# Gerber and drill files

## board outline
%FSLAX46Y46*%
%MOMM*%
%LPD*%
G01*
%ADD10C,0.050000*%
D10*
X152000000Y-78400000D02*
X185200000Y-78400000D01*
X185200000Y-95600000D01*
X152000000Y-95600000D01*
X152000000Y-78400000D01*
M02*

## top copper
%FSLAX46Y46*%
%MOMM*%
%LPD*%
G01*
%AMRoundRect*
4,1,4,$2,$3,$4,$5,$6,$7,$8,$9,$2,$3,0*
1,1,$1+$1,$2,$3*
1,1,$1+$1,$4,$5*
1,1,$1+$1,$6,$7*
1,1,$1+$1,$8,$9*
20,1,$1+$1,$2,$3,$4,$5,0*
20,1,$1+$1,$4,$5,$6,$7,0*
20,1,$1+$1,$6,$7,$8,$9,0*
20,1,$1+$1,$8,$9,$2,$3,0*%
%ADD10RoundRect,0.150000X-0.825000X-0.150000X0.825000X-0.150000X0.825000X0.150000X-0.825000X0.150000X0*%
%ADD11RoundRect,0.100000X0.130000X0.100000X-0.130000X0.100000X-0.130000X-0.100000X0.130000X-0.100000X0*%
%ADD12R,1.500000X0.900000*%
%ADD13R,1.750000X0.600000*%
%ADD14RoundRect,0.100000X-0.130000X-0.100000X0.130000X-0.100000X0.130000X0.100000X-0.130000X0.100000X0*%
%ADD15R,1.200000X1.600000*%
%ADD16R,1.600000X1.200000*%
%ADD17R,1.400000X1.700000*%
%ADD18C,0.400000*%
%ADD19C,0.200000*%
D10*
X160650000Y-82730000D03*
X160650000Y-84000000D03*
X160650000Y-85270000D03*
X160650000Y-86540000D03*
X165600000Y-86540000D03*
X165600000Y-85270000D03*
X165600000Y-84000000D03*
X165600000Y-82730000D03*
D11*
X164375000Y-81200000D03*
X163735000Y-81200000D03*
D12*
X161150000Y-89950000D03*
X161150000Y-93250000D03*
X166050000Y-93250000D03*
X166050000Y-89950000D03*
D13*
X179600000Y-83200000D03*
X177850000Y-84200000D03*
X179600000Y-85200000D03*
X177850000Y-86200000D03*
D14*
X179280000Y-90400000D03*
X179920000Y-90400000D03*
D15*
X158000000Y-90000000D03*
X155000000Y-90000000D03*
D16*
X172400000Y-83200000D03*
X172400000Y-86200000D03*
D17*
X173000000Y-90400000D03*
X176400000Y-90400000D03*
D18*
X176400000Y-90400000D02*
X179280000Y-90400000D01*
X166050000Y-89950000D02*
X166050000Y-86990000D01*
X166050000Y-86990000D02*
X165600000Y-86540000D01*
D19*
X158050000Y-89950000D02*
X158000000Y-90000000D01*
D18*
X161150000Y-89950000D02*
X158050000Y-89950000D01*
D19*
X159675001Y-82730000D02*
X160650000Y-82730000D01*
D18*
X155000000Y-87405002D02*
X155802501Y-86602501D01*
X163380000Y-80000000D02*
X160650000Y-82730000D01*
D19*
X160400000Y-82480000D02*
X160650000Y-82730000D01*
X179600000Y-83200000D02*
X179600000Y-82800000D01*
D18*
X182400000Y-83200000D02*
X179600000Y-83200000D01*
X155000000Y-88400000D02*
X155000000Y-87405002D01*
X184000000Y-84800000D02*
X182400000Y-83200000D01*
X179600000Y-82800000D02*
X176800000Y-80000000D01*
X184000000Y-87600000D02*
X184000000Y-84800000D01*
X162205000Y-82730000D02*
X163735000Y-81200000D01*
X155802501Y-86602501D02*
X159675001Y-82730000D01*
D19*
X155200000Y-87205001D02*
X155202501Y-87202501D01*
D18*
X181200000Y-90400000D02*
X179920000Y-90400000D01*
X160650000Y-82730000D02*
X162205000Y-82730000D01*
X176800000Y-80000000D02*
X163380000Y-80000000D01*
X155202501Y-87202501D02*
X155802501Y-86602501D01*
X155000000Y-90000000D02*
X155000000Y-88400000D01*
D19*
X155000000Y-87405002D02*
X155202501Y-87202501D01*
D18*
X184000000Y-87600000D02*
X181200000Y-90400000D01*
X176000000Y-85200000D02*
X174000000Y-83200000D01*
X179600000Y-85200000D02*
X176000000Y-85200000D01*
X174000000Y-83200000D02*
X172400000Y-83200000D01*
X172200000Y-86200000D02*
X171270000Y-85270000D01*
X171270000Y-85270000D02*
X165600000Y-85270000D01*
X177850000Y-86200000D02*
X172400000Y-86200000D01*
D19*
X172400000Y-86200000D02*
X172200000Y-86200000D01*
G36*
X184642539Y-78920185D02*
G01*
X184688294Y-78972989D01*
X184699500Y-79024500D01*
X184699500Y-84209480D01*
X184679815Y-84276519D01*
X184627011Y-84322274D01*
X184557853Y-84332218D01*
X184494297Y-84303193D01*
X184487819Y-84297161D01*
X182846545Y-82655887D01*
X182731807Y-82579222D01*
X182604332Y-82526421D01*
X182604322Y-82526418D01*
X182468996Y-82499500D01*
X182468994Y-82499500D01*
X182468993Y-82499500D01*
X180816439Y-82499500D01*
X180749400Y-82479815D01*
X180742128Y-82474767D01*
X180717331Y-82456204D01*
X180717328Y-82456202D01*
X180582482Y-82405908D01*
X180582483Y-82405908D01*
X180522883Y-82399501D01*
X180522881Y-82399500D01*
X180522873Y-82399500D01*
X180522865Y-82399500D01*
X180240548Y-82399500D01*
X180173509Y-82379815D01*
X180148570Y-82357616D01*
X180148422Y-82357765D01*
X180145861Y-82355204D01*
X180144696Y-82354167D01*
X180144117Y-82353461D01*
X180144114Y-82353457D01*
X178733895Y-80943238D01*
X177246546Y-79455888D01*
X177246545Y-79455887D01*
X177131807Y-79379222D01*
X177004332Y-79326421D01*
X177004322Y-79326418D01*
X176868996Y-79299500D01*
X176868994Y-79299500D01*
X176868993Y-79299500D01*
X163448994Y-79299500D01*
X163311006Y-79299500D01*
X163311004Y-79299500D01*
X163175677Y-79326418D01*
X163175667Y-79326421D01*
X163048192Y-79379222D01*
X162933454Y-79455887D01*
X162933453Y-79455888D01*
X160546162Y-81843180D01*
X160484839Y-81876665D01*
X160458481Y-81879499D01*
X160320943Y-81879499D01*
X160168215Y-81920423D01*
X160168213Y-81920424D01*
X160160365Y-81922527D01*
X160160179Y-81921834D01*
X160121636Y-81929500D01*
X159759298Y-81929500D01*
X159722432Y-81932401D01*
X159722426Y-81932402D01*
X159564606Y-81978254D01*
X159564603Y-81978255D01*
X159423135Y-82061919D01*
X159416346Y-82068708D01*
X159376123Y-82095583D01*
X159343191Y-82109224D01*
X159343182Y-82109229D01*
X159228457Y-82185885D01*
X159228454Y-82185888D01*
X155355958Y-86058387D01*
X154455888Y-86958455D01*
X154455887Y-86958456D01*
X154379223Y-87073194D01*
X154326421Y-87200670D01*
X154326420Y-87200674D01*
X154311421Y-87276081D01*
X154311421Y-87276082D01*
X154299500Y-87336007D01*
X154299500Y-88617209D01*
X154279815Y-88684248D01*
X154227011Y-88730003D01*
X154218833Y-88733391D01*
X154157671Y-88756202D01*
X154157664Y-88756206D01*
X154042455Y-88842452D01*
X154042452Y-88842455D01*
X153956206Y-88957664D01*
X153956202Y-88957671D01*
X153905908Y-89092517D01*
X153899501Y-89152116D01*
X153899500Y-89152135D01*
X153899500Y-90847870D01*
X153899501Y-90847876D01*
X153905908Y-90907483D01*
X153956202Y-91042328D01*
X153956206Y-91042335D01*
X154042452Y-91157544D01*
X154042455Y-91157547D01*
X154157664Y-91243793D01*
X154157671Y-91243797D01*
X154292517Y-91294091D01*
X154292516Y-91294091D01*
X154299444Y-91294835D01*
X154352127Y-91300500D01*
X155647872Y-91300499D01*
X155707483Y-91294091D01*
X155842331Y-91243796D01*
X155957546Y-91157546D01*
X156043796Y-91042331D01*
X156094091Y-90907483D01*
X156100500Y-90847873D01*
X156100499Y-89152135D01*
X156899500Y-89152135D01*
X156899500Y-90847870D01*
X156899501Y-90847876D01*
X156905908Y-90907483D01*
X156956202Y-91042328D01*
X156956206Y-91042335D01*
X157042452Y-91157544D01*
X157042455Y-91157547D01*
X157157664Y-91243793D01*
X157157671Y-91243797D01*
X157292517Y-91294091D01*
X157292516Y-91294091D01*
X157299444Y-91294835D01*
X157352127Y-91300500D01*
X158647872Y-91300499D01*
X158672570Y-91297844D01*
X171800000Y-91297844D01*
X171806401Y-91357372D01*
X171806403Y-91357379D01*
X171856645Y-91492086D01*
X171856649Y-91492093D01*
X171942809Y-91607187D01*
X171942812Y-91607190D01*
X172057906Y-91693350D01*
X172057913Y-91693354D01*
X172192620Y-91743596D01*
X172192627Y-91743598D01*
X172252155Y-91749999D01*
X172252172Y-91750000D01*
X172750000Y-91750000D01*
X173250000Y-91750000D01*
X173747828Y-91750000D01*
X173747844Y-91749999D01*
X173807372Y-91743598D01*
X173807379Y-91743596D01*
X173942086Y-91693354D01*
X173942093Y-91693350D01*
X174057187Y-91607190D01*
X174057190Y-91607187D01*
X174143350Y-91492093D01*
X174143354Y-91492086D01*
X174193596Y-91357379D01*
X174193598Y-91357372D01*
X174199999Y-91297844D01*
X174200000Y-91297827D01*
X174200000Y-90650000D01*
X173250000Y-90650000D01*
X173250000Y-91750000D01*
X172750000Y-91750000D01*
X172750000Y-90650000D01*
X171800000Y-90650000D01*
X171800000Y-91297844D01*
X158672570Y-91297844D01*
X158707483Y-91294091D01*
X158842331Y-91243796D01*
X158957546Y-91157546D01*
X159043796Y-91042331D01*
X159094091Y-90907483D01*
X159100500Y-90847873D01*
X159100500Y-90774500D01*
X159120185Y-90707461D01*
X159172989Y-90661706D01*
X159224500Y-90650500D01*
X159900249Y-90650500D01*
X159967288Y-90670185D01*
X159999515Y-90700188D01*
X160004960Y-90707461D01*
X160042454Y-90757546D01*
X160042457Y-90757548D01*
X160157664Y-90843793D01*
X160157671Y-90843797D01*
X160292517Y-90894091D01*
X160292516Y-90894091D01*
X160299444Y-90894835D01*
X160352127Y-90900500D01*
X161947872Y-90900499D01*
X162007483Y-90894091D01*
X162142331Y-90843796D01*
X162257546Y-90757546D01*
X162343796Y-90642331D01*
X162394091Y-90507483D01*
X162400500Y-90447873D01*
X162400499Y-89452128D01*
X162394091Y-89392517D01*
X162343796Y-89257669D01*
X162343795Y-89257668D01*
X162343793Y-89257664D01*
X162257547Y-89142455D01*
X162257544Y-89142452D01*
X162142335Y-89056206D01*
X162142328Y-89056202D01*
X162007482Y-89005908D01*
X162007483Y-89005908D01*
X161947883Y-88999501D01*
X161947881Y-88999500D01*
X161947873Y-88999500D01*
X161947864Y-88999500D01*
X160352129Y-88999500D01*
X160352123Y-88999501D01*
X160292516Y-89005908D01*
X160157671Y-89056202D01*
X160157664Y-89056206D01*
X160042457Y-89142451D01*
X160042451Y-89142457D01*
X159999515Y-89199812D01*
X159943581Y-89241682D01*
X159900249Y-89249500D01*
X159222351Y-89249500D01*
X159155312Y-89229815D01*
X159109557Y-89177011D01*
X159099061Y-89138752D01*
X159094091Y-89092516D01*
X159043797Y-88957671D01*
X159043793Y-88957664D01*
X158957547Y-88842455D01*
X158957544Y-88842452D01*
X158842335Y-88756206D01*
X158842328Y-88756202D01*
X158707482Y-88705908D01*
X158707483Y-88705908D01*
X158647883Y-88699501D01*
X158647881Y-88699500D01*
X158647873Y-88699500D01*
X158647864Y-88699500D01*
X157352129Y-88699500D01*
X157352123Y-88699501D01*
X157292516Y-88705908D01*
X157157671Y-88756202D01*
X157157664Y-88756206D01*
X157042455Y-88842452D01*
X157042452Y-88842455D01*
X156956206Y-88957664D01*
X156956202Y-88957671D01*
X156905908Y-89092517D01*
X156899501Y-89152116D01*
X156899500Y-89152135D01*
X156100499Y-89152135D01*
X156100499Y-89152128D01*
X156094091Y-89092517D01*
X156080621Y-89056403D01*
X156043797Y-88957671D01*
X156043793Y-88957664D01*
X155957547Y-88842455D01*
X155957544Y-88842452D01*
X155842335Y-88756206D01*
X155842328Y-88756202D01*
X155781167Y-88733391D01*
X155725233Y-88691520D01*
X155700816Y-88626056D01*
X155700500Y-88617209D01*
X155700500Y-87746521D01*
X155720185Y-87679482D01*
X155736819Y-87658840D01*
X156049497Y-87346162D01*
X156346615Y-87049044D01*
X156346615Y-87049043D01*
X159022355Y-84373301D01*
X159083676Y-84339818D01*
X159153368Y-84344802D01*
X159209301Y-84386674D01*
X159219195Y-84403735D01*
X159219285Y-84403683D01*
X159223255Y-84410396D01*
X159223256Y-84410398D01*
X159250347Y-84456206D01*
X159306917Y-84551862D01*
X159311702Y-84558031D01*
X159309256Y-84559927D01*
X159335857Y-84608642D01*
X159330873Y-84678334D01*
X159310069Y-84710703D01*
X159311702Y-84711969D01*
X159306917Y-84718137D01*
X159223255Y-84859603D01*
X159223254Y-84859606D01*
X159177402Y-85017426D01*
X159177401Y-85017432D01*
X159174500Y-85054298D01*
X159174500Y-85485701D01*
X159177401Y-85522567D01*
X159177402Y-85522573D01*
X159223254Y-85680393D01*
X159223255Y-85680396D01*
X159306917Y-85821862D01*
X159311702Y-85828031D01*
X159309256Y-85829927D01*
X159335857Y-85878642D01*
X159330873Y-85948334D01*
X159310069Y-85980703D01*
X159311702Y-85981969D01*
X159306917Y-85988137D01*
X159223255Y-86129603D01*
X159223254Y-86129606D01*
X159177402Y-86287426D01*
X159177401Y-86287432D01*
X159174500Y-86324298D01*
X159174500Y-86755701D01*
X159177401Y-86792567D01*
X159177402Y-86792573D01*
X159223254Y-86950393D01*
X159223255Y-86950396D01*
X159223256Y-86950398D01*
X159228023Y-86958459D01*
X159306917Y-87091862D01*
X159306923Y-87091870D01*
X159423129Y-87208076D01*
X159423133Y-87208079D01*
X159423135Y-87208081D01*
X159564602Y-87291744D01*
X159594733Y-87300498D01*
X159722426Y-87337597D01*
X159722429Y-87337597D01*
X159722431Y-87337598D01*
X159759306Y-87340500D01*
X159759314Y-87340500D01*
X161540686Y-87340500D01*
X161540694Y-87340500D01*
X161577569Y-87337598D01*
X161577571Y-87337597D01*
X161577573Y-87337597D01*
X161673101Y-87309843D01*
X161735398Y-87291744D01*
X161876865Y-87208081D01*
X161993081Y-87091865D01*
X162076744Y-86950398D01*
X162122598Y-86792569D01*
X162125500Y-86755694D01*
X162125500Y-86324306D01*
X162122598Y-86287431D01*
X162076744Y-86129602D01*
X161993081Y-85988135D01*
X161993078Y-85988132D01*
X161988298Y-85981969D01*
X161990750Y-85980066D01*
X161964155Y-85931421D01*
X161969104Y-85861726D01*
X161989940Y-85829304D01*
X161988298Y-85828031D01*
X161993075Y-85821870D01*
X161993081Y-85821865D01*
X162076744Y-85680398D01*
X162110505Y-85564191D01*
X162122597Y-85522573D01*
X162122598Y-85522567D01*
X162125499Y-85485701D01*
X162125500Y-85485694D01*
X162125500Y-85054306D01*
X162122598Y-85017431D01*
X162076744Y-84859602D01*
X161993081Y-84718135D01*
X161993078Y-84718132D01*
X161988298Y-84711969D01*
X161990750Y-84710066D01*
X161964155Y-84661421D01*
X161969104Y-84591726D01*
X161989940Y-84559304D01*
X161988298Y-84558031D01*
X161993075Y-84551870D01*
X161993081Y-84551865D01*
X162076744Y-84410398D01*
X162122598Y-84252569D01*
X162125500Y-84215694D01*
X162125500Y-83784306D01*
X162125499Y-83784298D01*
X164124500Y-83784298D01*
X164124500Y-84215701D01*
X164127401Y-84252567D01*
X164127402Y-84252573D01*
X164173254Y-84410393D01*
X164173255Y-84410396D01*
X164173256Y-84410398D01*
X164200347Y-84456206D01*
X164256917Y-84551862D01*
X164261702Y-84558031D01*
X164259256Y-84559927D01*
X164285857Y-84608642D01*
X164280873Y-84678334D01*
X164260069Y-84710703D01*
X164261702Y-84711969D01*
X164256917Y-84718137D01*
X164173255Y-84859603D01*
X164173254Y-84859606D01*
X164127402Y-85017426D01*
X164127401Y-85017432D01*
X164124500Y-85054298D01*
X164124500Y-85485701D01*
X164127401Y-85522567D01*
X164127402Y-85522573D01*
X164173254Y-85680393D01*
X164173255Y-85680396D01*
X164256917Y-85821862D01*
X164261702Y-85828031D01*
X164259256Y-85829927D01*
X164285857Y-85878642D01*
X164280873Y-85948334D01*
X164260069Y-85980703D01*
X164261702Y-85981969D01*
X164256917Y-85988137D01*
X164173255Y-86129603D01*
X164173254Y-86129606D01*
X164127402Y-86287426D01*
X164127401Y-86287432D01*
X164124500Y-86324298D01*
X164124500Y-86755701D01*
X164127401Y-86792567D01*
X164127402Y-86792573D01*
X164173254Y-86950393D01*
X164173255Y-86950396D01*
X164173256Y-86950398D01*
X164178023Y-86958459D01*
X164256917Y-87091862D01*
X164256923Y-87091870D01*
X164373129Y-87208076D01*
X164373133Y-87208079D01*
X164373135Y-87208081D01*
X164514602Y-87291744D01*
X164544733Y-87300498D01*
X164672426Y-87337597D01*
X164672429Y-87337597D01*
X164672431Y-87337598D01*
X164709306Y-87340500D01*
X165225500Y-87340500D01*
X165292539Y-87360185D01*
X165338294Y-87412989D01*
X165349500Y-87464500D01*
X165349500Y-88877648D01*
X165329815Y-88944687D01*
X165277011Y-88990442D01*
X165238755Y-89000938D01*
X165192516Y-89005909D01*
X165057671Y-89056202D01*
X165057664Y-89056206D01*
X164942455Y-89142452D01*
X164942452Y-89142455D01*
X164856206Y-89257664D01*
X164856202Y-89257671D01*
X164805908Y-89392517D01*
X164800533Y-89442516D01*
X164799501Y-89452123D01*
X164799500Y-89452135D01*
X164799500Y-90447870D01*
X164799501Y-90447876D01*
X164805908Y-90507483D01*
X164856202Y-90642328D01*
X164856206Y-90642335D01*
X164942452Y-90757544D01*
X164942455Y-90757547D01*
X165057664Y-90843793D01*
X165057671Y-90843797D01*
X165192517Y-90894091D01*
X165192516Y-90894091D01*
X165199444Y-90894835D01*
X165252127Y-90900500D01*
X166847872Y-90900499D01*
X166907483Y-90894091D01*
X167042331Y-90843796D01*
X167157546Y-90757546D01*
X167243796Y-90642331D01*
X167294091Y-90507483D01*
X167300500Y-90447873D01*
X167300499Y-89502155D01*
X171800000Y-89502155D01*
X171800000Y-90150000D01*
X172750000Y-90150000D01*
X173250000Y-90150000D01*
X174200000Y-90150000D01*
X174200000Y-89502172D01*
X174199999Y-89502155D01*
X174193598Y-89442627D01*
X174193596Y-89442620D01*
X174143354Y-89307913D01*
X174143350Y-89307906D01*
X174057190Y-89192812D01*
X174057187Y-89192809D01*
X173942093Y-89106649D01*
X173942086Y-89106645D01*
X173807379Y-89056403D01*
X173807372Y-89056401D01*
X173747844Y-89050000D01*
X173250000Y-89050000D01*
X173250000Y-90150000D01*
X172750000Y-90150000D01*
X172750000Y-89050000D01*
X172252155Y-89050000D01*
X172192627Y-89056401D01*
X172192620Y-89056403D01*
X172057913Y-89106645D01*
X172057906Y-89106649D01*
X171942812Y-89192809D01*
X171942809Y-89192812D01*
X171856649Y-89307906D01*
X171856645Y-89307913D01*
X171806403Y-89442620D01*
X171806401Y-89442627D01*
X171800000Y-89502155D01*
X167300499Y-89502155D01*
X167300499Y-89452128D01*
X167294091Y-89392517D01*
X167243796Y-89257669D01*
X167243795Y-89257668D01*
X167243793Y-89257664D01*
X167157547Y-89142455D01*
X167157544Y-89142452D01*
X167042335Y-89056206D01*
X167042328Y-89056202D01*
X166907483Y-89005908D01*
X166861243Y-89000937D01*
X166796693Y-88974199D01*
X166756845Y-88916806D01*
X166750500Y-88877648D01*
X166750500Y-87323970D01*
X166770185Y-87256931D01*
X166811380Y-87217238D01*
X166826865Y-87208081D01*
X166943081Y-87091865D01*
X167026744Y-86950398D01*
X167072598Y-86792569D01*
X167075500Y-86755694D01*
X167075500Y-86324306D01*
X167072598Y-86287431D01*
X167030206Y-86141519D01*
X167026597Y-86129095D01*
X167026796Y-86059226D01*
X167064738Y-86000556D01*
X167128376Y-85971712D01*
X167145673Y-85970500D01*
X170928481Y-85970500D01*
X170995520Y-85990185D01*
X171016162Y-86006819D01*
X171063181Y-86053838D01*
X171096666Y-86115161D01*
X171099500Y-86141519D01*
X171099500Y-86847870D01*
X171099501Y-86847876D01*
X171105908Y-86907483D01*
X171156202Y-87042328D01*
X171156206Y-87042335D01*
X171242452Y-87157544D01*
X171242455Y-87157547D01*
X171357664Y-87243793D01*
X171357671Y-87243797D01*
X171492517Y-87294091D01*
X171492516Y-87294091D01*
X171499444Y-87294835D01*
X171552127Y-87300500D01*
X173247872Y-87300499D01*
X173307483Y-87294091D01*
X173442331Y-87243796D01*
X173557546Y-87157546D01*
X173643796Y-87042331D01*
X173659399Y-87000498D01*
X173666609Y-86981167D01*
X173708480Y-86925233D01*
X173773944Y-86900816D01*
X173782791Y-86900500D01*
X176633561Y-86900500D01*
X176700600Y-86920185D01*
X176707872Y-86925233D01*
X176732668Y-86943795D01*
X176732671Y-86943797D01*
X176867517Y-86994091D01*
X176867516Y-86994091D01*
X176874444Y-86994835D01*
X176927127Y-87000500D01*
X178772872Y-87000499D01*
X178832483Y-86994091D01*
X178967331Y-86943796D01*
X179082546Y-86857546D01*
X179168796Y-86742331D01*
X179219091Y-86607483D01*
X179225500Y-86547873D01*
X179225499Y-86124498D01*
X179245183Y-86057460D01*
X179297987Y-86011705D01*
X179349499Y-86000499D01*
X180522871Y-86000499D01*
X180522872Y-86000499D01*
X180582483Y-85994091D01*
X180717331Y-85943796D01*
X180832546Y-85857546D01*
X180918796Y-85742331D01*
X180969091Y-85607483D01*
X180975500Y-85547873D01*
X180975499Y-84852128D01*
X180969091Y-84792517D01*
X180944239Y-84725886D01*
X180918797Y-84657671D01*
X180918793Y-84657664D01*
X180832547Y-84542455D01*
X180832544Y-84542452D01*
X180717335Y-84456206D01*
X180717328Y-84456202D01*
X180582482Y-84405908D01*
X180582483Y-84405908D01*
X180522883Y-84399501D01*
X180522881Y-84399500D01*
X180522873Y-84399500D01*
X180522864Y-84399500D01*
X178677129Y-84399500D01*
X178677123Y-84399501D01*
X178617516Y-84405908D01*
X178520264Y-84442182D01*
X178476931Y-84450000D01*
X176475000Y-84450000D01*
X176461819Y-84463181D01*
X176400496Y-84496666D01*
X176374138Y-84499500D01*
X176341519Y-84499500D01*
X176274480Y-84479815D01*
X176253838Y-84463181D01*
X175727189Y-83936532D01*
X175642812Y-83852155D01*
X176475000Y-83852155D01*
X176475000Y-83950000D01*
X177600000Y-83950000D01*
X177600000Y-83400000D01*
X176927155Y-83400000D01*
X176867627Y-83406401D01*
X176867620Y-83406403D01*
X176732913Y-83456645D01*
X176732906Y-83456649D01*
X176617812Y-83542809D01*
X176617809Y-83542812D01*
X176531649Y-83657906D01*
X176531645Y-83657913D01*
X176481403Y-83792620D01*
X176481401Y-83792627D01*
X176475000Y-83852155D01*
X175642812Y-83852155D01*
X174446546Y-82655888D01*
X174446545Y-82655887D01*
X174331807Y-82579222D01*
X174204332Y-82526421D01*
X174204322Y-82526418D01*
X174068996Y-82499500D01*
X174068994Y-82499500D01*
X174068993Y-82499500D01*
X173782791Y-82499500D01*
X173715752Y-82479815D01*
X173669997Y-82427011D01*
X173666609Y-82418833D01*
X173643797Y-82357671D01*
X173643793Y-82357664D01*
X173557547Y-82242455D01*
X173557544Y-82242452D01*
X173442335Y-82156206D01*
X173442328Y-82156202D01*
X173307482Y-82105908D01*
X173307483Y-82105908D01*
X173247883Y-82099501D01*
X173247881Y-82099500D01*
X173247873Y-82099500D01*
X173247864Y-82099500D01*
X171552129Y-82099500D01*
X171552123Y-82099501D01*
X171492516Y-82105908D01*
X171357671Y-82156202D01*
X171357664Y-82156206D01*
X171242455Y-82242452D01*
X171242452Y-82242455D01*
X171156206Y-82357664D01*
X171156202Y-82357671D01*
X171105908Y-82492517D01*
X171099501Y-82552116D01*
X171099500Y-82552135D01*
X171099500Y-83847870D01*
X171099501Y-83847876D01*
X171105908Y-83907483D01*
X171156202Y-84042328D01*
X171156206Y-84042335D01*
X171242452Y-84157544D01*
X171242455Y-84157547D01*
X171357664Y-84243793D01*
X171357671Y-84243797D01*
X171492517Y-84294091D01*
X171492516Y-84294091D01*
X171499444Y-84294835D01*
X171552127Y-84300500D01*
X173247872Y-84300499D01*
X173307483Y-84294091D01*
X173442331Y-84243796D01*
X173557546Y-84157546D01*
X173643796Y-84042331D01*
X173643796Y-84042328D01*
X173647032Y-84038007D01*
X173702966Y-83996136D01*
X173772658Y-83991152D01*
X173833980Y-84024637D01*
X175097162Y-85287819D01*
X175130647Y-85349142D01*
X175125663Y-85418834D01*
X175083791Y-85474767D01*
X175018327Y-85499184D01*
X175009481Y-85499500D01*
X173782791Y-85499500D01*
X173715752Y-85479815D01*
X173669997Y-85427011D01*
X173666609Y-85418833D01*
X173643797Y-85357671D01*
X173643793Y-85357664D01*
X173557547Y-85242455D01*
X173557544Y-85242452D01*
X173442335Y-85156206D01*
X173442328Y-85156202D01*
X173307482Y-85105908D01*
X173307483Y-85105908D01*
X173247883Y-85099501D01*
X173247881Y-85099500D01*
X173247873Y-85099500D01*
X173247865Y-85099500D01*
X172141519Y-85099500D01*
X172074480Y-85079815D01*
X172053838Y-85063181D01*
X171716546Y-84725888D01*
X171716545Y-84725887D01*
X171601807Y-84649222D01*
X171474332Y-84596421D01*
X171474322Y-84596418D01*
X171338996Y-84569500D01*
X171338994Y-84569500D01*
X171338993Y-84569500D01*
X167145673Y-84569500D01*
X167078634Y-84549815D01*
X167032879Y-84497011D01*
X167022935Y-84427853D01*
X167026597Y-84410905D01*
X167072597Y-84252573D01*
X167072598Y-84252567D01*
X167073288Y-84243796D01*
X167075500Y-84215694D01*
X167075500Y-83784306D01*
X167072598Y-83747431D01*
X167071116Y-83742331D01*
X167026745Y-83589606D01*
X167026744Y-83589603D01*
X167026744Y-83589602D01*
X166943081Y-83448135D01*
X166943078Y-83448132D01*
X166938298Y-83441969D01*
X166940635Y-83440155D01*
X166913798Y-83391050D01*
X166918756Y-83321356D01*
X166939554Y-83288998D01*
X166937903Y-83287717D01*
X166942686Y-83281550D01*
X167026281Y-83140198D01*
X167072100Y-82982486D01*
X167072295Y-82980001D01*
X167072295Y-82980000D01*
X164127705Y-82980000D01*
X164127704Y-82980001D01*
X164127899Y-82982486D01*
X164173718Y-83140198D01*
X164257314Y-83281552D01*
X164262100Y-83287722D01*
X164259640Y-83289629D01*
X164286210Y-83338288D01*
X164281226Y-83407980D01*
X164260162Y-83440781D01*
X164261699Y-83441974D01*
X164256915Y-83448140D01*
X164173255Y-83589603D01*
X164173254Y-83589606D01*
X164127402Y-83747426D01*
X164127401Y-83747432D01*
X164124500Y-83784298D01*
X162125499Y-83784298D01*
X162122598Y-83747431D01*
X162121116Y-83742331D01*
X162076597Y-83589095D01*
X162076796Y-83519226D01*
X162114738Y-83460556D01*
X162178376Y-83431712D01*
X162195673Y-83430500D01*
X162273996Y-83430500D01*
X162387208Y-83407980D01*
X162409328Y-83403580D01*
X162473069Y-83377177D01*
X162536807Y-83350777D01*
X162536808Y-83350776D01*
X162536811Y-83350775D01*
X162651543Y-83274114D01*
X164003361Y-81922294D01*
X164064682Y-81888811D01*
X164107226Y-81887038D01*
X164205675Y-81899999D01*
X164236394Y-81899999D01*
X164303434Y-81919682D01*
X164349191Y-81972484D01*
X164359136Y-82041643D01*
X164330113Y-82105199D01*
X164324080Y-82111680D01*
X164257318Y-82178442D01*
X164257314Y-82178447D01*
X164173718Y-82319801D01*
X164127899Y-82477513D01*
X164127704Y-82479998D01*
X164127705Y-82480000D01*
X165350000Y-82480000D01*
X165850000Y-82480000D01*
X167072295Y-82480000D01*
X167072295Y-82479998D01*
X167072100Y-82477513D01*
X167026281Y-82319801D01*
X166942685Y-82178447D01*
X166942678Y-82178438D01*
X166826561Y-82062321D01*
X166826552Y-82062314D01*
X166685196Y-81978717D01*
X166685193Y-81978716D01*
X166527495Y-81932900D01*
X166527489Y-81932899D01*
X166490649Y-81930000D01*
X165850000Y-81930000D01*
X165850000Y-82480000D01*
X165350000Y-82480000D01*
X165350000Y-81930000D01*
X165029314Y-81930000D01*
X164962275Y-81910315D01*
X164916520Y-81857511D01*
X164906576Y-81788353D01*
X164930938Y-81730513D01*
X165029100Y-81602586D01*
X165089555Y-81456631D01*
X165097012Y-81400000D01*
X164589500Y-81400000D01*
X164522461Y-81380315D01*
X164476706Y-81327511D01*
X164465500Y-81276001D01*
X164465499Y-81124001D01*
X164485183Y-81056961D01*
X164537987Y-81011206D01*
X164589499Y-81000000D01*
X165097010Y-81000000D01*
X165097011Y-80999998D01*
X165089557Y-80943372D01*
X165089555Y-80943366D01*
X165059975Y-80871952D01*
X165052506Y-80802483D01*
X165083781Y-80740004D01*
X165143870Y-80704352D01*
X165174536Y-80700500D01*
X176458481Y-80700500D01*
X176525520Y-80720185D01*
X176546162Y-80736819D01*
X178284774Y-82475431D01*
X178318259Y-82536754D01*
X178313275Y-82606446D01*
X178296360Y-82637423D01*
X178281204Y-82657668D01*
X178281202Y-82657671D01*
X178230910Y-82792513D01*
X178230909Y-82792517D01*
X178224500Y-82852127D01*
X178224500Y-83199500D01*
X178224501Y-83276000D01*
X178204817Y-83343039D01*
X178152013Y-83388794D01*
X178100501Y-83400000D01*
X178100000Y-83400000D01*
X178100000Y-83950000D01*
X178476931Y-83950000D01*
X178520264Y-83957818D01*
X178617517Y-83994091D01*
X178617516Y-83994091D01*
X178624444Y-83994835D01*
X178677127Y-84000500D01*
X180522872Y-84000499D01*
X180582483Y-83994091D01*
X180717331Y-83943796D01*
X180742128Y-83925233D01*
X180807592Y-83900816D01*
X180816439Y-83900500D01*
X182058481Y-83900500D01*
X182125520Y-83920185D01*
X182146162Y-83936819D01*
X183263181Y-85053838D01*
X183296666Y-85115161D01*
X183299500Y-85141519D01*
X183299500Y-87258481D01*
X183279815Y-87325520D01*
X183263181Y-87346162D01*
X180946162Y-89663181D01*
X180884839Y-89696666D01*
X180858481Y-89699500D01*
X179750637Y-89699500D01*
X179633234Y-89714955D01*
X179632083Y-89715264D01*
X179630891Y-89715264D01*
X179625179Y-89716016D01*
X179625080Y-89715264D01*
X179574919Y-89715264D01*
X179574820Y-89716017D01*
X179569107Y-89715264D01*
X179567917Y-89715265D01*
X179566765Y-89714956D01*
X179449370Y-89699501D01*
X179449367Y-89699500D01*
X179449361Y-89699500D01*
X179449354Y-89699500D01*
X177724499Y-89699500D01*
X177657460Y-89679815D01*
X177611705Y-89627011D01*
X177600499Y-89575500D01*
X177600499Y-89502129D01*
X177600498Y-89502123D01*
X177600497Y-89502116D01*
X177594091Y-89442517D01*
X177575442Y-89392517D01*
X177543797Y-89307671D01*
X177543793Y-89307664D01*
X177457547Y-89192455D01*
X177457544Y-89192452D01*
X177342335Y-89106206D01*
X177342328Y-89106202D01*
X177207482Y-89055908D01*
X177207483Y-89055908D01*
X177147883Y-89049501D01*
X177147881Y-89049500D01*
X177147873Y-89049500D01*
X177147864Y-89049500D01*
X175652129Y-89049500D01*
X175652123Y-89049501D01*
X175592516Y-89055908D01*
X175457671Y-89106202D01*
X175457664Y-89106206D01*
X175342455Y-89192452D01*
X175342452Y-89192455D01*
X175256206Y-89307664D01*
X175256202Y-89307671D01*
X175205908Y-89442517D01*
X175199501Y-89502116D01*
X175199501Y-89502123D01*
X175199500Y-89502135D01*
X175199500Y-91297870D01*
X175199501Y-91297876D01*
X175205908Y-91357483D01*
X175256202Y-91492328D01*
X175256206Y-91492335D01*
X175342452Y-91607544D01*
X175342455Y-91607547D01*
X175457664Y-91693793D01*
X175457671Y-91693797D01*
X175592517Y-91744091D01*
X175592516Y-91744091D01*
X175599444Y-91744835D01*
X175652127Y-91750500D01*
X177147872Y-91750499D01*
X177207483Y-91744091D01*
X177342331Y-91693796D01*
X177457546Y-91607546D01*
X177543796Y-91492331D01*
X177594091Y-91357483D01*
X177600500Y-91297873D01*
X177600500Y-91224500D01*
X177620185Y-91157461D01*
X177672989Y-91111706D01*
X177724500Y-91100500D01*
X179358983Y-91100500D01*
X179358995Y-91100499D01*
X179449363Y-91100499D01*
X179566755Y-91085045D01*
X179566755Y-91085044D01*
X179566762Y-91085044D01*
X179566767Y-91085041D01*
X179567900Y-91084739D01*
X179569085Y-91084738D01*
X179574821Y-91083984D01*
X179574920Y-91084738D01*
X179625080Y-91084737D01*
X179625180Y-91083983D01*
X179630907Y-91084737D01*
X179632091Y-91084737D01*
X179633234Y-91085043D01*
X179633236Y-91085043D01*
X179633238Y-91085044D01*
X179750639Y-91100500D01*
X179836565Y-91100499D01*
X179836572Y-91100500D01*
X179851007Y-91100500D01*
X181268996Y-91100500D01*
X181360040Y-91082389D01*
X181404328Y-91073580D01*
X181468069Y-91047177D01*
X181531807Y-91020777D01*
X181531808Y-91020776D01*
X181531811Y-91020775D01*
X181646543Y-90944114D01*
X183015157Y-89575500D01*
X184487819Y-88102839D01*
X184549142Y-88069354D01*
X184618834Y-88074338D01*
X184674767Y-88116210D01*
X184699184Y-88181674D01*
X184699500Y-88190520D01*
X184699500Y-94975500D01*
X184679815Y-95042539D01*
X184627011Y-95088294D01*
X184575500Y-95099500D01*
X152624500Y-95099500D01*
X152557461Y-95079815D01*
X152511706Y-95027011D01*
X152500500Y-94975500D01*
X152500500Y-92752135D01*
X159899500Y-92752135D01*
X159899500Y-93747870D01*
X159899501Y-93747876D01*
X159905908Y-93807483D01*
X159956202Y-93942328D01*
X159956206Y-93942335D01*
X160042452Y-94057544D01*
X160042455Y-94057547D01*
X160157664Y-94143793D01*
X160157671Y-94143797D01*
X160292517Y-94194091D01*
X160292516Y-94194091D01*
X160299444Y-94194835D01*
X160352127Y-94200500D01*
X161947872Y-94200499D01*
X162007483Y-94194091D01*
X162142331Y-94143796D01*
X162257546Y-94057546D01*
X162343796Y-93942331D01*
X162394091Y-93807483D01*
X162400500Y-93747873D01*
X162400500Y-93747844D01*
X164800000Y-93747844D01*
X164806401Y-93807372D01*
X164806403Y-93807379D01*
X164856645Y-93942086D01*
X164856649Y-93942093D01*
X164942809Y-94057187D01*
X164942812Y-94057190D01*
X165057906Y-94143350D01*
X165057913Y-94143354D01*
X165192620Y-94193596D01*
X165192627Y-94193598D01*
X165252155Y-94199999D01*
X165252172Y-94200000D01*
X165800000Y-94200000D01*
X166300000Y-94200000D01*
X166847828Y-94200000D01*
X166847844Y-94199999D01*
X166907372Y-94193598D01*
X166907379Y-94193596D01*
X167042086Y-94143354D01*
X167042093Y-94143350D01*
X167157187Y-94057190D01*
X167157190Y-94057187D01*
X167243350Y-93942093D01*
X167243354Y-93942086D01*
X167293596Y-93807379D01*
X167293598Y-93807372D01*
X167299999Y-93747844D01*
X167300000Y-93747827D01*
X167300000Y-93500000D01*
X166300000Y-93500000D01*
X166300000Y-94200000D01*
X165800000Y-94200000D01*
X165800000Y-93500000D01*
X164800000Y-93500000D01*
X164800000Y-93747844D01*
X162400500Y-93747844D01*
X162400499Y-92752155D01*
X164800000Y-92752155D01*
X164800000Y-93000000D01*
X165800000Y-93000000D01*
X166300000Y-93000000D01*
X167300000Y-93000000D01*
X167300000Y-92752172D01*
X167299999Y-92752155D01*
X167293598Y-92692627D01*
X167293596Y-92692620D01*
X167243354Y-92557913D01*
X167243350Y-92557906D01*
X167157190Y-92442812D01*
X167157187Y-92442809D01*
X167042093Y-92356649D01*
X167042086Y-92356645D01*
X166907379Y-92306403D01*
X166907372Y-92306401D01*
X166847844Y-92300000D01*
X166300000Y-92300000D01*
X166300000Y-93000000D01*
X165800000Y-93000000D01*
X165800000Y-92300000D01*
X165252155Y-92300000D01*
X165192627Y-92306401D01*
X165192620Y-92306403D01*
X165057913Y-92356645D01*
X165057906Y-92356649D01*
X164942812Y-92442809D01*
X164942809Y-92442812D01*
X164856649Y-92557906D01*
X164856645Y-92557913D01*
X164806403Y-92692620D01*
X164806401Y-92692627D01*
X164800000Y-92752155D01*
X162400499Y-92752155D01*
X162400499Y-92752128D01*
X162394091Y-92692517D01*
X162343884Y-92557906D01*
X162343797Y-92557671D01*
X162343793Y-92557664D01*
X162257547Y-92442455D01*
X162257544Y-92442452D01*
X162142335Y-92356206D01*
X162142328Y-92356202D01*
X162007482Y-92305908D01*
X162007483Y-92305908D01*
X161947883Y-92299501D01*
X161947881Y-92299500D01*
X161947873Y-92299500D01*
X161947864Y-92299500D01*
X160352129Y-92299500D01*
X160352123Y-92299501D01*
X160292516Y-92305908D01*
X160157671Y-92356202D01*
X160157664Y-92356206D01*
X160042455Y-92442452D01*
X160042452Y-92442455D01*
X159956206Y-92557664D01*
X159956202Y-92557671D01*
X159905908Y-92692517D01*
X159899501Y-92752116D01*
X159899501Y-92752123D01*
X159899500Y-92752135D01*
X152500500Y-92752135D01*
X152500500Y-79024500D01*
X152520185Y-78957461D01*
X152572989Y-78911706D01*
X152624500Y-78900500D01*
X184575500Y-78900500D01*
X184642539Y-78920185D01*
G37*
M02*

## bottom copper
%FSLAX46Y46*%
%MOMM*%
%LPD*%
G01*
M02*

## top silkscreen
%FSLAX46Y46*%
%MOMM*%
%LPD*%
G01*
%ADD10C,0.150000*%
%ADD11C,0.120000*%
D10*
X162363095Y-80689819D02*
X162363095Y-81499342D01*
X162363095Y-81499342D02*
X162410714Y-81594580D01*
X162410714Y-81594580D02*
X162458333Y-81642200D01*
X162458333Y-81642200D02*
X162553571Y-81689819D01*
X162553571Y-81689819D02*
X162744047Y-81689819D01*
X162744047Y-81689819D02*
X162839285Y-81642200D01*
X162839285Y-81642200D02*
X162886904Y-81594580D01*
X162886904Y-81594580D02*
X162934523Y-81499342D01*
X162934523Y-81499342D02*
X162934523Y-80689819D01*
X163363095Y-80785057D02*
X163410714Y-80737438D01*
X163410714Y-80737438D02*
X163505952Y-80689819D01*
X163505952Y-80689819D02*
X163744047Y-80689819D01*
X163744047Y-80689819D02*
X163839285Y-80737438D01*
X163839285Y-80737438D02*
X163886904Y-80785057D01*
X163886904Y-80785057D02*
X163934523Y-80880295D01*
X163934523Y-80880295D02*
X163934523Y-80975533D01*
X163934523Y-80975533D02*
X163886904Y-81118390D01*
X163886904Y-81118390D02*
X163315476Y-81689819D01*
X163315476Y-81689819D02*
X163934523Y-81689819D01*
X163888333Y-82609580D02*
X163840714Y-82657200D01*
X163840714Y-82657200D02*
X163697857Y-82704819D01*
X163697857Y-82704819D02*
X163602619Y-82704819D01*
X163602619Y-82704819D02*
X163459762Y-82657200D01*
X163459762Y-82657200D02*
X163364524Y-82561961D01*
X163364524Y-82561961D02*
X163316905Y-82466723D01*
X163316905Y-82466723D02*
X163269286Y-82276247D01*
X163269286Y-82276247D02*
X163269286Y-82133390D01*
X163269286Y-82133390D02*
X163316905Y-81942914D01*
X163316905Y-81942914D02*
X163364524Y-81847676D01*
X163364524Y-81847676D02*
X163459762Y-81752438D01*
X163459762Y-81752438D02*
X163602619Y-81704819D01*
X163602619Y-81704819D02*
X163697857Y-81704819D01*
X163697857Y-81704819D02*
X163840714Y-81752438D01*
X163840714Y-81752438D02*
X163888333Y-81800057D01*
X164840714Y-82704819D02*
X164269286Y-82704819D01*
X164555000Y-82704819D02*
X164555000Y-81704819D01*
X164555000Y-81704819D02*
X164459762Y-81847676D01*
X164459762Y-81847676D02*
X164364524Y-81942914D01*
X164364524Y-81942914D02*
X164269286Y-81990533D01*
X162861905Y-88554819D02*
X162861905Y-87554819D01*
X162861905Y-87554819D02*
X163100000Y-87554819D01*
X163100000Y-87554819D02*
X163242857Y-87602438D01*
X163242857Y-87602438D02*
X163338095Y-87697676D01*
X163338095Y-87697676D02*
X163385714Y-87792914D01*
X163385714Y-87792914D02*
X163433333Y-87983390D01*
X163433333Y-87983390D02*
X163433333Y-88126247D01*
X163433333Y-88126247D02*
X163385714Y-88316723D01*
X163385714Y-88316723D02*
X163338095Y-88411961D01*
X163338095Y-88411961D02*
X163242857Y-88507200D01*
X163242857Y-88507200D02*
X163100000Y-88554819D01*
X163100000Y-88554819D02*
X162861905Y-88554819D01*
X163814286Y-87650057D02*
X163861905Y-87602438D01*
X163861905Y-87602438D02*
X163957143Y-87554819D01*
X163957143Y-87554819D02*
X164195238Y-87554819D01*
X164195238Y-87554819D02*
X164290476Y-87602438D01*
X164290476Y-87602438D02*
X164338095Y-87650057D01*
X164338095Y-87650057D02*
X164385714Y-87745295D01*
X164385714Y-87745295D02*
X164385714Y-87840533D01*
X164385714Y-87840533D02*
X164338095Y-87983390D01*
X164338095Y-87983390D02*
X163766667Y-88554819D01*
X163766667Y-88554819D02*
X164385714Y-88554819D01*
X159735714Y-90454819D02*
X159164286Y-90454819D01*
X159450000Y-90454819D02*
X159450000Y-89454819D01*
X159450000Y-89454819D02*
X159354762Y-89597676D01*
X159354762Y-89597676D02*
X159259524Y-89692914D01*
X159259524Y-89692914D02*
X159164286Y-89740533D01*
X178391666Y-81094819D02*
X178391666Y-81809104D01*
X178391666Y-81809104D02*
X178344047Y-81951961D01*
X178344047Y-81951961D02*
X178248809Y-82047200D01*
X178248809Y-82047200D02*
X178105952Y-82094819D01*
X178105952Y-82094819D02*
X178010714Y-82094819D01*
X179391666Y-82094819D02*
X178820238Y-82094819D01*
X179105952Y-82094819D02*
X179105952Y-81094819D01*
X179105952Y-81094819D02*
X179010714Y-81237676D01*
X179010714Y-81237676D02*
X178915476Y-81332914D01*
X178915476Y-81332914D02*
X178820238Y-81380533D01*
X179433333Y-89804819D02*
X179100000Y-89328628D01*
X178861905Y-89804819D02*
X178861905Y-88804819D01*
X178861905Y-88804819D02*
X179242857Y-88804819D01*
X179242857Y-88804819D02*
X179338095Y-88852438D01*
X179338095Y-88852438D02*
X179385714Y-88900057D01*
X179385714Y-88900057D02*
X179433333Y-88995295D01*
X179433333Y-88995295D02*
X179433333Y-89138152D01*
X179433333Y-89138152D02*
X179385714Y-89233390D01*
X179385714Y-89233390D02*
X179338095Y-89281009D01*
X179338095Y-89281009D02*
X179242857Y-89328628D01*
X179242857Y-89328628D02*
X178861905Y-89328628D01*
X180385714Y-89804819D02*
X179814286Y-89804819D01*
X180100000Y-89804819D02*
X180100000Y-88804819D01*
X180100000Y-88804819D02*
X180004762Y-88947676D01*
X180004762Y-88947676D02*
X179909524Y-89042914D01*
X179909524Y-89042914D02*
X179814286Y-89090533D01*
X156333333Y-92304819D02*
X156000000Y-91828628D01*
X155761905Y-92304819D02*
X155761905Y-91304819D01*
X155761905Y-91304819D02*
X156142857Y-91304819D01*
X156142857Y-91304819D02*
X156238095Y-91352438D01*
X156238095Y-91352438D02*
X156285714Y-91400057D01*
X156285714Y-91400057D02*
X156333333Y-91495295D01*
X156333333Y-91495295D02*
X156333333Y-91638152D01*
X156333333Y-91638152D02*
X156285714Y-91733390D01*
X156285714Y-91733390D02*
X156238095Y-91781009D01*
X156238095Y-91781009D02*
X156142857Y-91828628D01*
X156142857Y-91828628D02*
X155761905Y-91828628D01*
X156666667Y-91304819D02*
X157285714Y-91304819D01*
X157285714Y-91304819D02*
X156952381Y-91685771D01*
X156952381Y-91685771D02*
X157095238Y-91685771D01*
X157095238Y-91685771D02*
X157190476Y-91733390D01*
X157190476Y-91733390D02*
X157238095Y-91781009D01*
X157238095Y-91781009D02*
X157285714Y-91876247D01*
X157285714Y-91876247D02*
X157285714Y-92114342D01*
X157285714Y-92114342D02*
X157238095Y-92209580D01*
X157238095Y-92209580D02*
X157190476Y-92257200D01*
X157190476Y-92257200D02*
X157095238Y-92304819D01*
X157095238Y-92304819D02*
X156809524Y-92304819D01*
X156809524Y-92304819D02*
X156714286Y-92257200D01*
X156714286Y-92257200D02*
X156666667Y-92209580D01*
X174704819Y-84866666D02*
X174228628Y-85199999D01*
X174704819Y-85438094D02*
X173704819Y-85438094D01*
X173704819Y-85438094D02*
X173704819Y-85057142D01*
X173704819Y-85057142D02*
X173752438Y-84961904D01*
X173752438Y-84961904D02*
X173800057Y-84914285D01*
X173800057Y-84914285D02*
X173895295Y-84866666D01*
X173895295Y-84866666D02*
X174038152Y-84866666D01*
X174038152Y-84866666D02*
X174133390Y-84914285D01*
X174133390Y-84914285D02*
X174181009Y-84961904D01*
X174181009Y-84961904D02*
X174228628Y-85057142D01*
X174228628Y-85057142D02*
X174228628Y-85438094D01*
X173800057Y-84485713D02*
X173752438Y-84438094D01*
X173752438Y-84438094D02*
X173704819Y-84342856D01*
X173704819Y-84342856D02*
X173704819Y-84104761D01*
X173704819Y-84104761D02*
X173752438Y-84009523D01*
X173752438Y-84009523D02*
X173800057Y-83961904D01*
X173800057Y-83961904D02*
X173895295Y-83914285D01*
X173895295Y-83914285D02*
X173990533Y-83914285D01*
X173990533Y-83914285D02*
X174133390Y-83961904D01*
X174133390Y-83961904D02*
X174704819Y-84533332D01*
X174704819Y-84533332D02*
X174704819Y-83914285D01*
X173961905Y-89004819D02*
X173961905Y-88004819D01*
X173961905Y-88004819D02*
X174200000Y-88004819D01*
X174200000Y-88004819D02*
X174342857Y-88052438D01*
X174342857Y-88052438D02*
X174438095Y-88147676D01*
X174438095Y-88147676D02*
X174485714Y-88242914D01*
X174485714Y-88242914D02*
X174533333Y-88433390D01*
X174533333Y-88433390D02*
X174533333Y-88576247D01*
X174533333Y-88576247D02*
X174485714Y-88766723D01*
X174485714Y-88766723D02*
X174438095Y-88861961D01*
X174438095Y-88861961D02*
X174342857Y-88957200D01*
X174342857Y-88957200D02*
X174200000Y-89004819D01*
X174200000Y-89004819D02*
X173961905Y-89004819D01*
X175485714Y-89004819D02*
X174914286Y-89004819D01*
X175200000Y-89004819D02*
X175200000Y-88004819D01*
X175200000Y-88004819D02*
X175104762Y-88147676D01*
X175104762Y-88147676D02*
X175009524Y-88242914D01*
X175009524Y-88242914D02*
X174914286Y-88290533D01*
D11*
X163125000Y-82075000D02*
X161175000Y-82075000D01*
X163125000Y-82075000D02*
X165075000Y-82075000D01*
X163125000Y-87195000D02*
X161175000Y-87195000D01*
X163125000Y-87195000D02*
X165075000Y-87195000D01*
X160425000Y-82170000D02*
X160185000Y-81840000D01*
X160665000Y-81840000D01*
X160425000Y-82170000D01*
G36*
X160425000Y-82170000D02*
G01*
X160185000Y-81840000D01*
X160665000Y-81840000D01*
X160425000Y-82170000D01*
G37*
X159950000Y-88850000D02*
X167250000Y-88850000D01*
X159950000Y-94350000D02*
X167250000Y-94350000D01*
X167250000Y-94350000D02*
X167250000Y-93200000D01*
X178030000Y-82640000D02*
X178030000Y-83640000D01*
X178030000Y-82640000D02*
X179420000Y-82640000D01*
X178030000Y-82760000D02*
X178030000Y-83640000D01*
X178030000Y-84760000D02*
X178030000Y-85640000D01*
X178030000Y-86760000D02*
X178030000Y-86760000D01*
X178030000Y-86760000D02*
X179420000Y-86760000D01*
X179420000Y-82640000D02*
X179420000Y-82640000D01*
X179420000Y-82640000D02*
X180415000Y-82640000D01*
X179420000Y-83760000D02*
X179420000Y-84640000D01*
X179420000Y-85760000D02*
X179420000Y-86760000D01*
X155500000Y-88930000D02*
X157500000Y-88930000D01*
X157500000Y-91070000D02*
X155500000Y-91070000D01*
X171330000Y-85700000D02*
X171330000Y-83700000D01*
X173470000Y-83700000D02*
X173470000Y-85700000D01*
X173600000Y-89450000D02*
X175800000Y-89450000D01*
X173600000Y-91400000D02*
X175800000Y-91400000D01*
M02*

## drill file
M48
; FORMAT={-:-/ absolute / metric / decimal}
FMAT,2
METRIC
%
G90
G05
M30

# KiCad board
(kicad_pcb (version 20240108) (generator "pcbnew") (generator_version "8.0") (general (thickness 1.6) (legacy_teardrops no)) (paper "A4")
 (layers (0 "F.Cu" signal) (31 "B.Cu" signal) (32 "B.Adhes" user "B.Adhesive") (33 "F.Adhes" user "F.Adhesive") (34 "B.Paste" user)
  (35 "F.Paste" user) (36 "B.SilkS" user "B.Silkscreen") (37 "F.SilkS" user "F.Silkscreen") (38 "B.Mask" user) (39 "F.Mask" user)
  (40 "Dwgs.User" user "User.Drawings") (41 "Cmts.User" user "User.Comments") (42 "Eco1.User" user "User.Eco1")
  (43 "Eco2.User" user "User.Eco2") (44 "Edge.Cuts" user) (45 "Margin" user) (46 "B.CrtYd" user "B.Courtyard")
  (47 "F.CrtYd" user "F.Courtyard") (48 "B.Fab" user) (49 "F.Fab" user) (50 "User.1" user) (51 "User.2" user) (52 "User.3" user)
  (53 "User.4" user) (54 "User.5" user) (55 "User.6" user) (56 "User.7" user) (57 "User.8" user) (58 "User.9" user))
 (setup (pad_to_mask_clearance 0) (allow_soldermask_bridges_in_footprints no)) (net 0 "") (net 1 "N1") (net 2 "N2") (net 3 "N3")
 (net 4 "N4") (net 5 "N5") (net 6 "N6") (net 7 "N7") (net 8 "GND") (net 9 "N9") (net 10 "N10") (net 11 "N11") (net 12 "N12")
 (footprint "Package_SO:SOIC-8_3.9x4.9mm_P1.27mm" (layer "F.Cu") (at 163.125 84.635)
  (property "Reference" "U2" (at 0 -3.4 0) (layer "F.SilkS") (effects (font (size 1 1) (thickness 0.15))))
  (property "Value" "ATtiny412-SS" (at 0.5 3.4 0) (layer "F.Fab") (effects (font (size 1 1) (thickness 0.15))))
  (fp_line (start 0 -2.56) (end -1.95 -2.56) (stroke (width 0.12) (type solid)) (layer "F.SilkS"))
  (fp_line (start 0 -2.56) (end 1.95 -2.56) (stroke (width 0.12) (type solid)) (layer "F.SilkS"))
  (fp_line (start 0 2.56) (end -1.95 2.56) (stroke (width 0.12) (type solid)) (layer "F.SilkS"))
  (fp_line (start 0 2.56) (end 1.95 2.56) (stroke (width 0.12) (type solid)) (layer "F.SilkS"))
  (fp_poly
   (pts (xy -2.7 -2.465) (xy -2.94 -2.795) (xy -2.46 -2.795) (xy -2.7 -2.465)) (stroke (width 0.12) (type solid)) (fill solid)
   (layer "F.SilkS"))
  (pad "1" smd roundrect (at -2.475 -1.905) (size 1.95 0.6) (layers "F.Cu" "F.Paste" "F.Mask") (roundrect_rratio 0.25) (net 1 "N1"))
  (pad "2" smd roundrect (at -2.475 -0.635) (size 1.95 0.6) (layers "F.Cu" "F.Paste" "F.Mask") (roundrect_rratio 0.25) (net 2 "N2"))
  (pad "3" smd roundrect (at -2.475 0.635) (size 1.95 0.6) (layers "F.Cu" "F.Paste" "F.Mask") (roundrect_rratio 0.25) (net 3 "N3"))
  (pad "4" smd roundrect (at -2.475 1.905) (size 1.95 0.6) (layers "F.Cu" "F.Paste" "F.Mask") (roundrect_rratio 0.25) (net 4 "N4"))
  (pad "5" smd roundrect (at 2.475 1.905) (size 1.95 0.6) (layers "F.Cu" "F.Paste" "F.Mask") (roundrect_rratio 0.25) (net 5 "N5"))
  (pad "6" smd roundrect (at 2.475 0.635) (size 1.95 0.6) (layers "F.Cu" "F.Paste" "F.Mask") (roundrect_rratio 0.25) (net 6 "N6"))
  (pad "7" smd roundrect (at 2.475 -0.635) (size 1.95 0.6) (layers "F.Cu" "F.Paste" "F.Mask") (roundrect_rratio 0.25) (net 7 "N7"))
  (pad "8" smd roundrect (at 2.475 -1.905) (size 1.95 0.6) (layers "F.Cu" "F.Paste" "F.Mask") (roundrect_rratio 0.25) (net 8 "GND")))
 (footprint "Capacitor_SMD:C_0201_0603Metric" (layer "F.Cu") (at 164.055 81.2 180)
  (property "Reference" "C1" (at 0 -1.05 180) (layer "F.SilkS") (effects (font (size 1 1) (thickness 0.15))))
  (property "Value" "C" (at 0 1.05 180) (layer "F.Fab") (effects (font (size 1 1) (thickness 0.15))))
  (pad "" smd roundrect (at -0.345 0 180) (size 0.318 0.36) (layers "F.Paste") (roundrect_rratio 0.25))
  (pad "" smd roundrect (at 0.345 0 180) (size 0.318 0.36) (layers "F.Paste") (roundrect_rratio 0.25))
  (pad "1" smd roundrect (at -0.32 0 180) (size 0.46 0.4) (layers "F.Cu" "F.Mask") (roundrect_rratio 0.25) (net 8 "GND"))
  (pad "2" smd roundrect (at 0.32 0 180) (size 0.46 0.4) (layers "F.Cu" "F.Mask") (roundrect_rratio 0.25) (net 1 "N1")))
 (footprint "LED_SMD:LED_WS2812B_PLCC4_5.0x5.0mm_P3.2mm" (layer "F.Cu") (at 163.6 91.6)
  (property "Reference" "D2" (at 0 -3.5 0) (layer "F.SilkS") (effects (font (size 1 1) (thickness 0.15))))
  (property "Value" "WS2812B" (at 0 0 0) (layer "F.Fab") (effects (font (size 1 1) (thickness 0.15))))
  (fp_line (start -3.65 -2.75) (end 3.65 -2.75) (stroke (width 0.12) (type solid)) (layer "F.SilkS"))
  (fp_line (start -3.65 2.75) (end 3.65 2.75) (stroke (width 0.12) (type solid)) (layer "F.SilkS"))
  (fp_line (start 3.65 2.75) (end 3.65 1.6) (stroke (width 0.12) (type solid)) (layer "F.SilkS"))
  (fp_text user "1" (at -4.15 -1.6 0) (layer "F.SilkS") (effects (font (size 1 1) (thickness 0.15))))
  (pad "1" smd rect (at -2.45 -1.65) (size 1.5 0.9) (layers "F.Cu" "F.Paste" "F.Mask") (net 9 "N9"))
  (pad "2" smd rect (at -2.45 1.65) (size 1.5 0.9) (layers "F.Cu" "F.Paste" "F.Mask") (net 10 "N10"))
  (pad "3" smd rect (at 2.45 1.65) (size 1.5 0.9) (layers "F.Cu" "F.Paste" "F.Mask") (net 8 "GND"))
  (pad "4" smd rect (at 2.45 -1.65) (size 1.5 0.9) (layers "F.Cu" "F.Paste" "F.Mask") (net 5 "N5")))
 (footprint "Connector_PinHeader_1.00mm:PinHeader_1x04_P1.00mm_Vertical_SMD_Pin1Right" (layer "F.Cu") (at 178.725 84.7)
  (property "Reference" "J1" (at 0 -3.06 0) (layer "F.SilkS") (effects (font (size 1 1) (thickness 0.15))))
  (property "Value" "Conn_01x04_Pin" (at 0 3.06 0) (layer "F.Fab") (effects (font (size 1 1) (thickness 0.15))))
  (fp_line (start -0.695 -2.06) (end -0.695 -1.06) (stroke (width 0.12) (type solid)) (layer "F.SilkS"))
  (fp_line (start -0.695 -2.06) (end 0.695 -2.06) (stroke (width 0.12) (type solid)) (layer "F.SilkS"))
  (fp_line (start -0.695 -1.94) (end -0.695 -1.06) (stroke (width 0.12) (type solid)) (layer "F.SilkS"))
  (fp_line (start -0.695 0.06) (end -0.695 0.94) (stroke (width 0.12) (type solid)) (layer "F.SilkS"))
  (fp_line (start -0.695 2.06) (end -0.695 2.06) (stroke (width 0.12) (type solid)) (layer "F.SilkS"))
  (fp_line (start -0.695 2.06) (end 0.695 2.06) (stroke (width 0.12) (type solid)) (layer "F.SilkS"))
  (fp_line (start 0.695 -2.06) (end 0.695 -2.06) (stroke (width 0.12) (type solid)) (layer "F.SilkS"))
  (fp_line (start 0.695 -2.06) (end 1.69 -2.06) (stroke (width 0.12) (type solid)) (layer "F.SilkS"))
  (fp_line (start 0.695 -0.94) (end 0.695 -0.06) (stroke (width 0.12) (type solid)) (layer "F.SilkS"))
  (fp_line (start 0.695 1.06) (end 0.695 2.06) (stroke (width 0.12) (type solid)) (layer "F.SilkS"))
  (pad "1" smd rect (at 0.875 -1.5) (size 1.75 0.6) (layers "F.Cu" "F.Paste" "F.Mask") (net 1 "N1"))
  (pad "2" smd rect (at -0.875 -0.5) (size 1.75 0.6) (layers "F.Cu" "F.Paste" "F.Mask") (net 8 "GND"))
  (pad "3" smd rect (at 0.875 0.5) (size 1.75 0.6) (layers "F.Cu" "F.Paste" "F.Mask") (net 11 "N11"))
  (pad "4" smd rect (at -0.875 1.5) (size 1.75 0.6) (layers "F.Cu" "F.Paste" "F.Mask") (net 6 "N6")))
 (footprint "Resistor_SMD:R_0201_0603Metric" (layer "F.Cu") (at 179.6 90.4)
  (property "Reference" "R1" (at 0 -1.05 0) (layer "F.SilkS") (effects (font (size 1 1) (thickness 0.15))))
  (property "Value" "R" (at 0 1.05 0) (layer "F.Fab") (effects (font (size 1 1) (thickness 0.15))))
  (pad "" smd roundrect (at -0.345 0) (size 0.318 0.36) (layers "F.Paste") (roundrect_rratio 0.25))
  (pad "" smd roundrect (at 0.345 0) (size 0.318 0.36) (layers "F.Paste") (roundrect_rratio 0.25))
  (pad "1" smd roundrect (at -0.32 0) (size 0.46 0.4) (layers "F.Cu" "F.Mask") (roundrect_rratio 0.25) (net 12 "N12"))
  (pad "2" smd roundrect (at 0.32 0) (size 0.46 0.4) (layers "F.Cu" "F.Mask") (roundrect_rratio 0.25) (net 1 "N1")))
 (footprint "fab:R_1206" (layer "F.Cu") (at 156.5 90 180)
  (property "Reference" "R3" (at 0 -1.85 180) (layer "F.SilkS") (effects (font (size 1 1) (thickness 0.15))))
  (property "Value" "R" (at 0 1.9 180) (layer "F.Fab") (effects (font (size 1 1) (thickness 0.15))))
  (fp_line (start 1 1.07) (end -1 1.07) (stroke (width 0.12) (type solid)) (layer "F.SilkS"))
  (fp_line (start -1 -1.07) (end 1 -1.07) (stroke (width 0.12) (type solid)) (layer "F.SilkS"))
  (pad "1" smd rect (at -1.5 0 180) (size 1.2 1.6) (layers "F.Cu" "F.Paste" "F.Mask") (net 9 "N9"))
  (pad "2" smd rect (at 1.5 0 180) (size 1.2 1.6) (layers "F.Cu" "F.Paste" "F.Mask") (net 1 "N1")))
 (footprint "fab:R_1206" (layer "F.Cu") (at 172.4 84.7 -90)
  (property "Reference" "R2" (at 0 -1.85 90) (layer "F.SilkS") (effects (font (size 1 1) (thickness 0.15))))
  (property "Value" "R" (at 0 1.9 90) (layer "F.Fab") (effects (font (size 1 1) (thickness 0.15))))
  (fp_line (start 1 1.07) (end -1 1.07) (stroke (width 0.12) (type solid)) (layer "F.SilkS"))
  (fp_line (start -1 -1.07) (end 1 -1.07) (stroke (width 0.12) (type solid)) (layer "F.SilkS"))
  (pad "1" smd rect (at -1.5 0 270) (size 1.2 1.6) (layers "F.Cu" "F.Paste" "F.Mask") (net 11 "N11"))
  (pad "2" smd rect (at 1.5 0 270) (size 1.2 1.6) (layers "F.Cu" "F.Paste" "F.Mask") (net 6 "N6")))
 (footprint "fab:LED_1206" (layer "F.Cu") (at 174.7 90.4)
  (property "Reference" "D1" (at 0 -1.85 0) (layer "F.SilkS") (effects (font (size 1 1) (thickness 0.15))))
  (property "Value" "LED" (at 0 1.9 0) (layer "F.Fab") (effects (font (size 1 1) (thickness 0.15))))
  (fp_line (start -1.1 -0.95) (end 1.1 -0.95) (stroke (width 0.12) (type solid)) (layer "F.SilkS"))
  (fp_line (start -1.1 1) (end 1.1 1) (stroke (width 0.12) (type solid)) (layer "F.SilkS"))
  (pad "1" smd rect (at -1.7 0) (size 1.4 1.7) (layers "F.Cu" "F.Paste" "F.Mask") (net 8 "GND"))
  (pad "2" smd rect (at 1.7 0) (size 1.4 1.7) (layers "F.Cu" "F.Paste" "F.Mask") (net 12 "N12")))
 (gr_rect (start 152 78.4) (end 185.2 95.6) (stroke (width 0.05) (type default)) (fill none) (layer "Edge.Cuts"))
 (segment (start 176.4 90.4) (end 179.28 90.4) (width 0.4) (layer "F.Cu") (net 12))
 (segment (start 166.05 89.95) (end 166.05 86.99) (width 0.4) (layer "F.Cu") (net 5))
 (segment (start 166.05 86.99) (end 165.6 86.54) (width 0.4) (layer "F.Cu") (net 5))
 (segment (start 158.05 89.95) (end 158 90) (width 0.2) (layer "F.Cu") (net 9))
 (segment (start 161.15 89.95) (end 158.05 89.95) (width 0.4) (layer "F.Cu") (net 9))
 (segment (start 159.675001 82.73) (end 160.65 82.73) (width 0.2) (layer "F.Cu") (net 1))
 (segment (start 155 87.405002) (end 155.802501 86.602501) (width 0.4) (layer "F.Cu") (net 1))
 (segment (start 163.38 80) (end 160.65 82.73) (width 0.4) (layer "F.Cu") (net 1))
 (segment (start 160.4 82.48) (end 160.65 82.73) (width 0.2) (layer "F.Cu") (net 1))
 (segment (start 179.6 83.2) (end 179.6 82.8) (width 0.2) (layer "F.Cu") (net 1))
 (segment (start 182.4 83.2) (end 179.6 83.2) (width 0.4) (layer "F.Cu") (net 1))
 (segment (start 155 88.4) (end 155 87.405002) (width 0.4) (layer "F.Cu") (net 1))
 (segment (start 184 84.8) (end 182.4 83.2) (width 0.4) (layer "F.Cu") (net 1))
 (segment (start 179.6 82.8) (end 176.8 80) (width 0.4) (layer "F.Cu") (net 1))
 (segment (start 184 87.6) (end 184 84.8) (width 0.4) (layer "F.Cu") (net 1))
 (segment (start 162.205 82.73) (end 163.735 81.2) (width 0.4) (layer "F.Cu") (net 1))
 (segment (start 155.802501 86.602501) (end 159.675001 82.73) (width 0.4) (layer "F.Cu") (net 1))
 (segment (start 155.2 87.205001) (end 155.202501 87.202501) (width 0.2) (layer "F.Cu") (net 1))
 (segment (start 181.2 90.4) (end 179.92 90.4) (width 0.4) (layer "F.Cu") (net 1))
 (segment (start 160.65 82.73) (end 162.205 82.73) (width 0.4) (layer "F.Cu") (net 1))
 (segment (start 176.8 80) (end 163.38 80) (width 0.4) (layer "F.Cu") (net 1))
 (segment (start 155.202501 87.202501) (end 155.802501 86.602501) (width 0.4) (layer "F.Cu") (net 1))
 (segment (start 155 90) (end 155 88.4) (width 0.4) (layer "F.Cu") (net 1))
 (segment (start 155 87.405002) (end 155.202501 87.202501) (width 0.2) (layer "F.Cu") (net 1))
 (segment (start 184 87.6) (end 181.2 90.4) (width 0.4) (layer "F.Cu") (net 1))
 (segment (start 176 85.2) (end 174 83.2) (width 0.4) (layer "F.Cu") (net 11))
 (segment (start 179.6 85.2) (end 176 85.2) (width 0.4) (layer "F.Cu") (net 11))
 (segment (start 174 83.2) (end 172.4 83.2) (width 0.4) (layer "F.Cu") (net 11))
 (segment (start 172.2 86.2) (end 171.27 85.27) (width 0.4) (layer "F.Cu") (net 6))
 (segment (start 171.27 85.27) (end 165.6 85.27) (width 0.4) (layer "F.Cu") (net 6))
 (segment (start 177.85 86.2) (end 172.4 86.2) (width 0.4) (layer "F.Cu") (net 6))
 (segment (start 172.4 86.2) (end 172.2 86.2) (width 0.2) (layer "F.Cu") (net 6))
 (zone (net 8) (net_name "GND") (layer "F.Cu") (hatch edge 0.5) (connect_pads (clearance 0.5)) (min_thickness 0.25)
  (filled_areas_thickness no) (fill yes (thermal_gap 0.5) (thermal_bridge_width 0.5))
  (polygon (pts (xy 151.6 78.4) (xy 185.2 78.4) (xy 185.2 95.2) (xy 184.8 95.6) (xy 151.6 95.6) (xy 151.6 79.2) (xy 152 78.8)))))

